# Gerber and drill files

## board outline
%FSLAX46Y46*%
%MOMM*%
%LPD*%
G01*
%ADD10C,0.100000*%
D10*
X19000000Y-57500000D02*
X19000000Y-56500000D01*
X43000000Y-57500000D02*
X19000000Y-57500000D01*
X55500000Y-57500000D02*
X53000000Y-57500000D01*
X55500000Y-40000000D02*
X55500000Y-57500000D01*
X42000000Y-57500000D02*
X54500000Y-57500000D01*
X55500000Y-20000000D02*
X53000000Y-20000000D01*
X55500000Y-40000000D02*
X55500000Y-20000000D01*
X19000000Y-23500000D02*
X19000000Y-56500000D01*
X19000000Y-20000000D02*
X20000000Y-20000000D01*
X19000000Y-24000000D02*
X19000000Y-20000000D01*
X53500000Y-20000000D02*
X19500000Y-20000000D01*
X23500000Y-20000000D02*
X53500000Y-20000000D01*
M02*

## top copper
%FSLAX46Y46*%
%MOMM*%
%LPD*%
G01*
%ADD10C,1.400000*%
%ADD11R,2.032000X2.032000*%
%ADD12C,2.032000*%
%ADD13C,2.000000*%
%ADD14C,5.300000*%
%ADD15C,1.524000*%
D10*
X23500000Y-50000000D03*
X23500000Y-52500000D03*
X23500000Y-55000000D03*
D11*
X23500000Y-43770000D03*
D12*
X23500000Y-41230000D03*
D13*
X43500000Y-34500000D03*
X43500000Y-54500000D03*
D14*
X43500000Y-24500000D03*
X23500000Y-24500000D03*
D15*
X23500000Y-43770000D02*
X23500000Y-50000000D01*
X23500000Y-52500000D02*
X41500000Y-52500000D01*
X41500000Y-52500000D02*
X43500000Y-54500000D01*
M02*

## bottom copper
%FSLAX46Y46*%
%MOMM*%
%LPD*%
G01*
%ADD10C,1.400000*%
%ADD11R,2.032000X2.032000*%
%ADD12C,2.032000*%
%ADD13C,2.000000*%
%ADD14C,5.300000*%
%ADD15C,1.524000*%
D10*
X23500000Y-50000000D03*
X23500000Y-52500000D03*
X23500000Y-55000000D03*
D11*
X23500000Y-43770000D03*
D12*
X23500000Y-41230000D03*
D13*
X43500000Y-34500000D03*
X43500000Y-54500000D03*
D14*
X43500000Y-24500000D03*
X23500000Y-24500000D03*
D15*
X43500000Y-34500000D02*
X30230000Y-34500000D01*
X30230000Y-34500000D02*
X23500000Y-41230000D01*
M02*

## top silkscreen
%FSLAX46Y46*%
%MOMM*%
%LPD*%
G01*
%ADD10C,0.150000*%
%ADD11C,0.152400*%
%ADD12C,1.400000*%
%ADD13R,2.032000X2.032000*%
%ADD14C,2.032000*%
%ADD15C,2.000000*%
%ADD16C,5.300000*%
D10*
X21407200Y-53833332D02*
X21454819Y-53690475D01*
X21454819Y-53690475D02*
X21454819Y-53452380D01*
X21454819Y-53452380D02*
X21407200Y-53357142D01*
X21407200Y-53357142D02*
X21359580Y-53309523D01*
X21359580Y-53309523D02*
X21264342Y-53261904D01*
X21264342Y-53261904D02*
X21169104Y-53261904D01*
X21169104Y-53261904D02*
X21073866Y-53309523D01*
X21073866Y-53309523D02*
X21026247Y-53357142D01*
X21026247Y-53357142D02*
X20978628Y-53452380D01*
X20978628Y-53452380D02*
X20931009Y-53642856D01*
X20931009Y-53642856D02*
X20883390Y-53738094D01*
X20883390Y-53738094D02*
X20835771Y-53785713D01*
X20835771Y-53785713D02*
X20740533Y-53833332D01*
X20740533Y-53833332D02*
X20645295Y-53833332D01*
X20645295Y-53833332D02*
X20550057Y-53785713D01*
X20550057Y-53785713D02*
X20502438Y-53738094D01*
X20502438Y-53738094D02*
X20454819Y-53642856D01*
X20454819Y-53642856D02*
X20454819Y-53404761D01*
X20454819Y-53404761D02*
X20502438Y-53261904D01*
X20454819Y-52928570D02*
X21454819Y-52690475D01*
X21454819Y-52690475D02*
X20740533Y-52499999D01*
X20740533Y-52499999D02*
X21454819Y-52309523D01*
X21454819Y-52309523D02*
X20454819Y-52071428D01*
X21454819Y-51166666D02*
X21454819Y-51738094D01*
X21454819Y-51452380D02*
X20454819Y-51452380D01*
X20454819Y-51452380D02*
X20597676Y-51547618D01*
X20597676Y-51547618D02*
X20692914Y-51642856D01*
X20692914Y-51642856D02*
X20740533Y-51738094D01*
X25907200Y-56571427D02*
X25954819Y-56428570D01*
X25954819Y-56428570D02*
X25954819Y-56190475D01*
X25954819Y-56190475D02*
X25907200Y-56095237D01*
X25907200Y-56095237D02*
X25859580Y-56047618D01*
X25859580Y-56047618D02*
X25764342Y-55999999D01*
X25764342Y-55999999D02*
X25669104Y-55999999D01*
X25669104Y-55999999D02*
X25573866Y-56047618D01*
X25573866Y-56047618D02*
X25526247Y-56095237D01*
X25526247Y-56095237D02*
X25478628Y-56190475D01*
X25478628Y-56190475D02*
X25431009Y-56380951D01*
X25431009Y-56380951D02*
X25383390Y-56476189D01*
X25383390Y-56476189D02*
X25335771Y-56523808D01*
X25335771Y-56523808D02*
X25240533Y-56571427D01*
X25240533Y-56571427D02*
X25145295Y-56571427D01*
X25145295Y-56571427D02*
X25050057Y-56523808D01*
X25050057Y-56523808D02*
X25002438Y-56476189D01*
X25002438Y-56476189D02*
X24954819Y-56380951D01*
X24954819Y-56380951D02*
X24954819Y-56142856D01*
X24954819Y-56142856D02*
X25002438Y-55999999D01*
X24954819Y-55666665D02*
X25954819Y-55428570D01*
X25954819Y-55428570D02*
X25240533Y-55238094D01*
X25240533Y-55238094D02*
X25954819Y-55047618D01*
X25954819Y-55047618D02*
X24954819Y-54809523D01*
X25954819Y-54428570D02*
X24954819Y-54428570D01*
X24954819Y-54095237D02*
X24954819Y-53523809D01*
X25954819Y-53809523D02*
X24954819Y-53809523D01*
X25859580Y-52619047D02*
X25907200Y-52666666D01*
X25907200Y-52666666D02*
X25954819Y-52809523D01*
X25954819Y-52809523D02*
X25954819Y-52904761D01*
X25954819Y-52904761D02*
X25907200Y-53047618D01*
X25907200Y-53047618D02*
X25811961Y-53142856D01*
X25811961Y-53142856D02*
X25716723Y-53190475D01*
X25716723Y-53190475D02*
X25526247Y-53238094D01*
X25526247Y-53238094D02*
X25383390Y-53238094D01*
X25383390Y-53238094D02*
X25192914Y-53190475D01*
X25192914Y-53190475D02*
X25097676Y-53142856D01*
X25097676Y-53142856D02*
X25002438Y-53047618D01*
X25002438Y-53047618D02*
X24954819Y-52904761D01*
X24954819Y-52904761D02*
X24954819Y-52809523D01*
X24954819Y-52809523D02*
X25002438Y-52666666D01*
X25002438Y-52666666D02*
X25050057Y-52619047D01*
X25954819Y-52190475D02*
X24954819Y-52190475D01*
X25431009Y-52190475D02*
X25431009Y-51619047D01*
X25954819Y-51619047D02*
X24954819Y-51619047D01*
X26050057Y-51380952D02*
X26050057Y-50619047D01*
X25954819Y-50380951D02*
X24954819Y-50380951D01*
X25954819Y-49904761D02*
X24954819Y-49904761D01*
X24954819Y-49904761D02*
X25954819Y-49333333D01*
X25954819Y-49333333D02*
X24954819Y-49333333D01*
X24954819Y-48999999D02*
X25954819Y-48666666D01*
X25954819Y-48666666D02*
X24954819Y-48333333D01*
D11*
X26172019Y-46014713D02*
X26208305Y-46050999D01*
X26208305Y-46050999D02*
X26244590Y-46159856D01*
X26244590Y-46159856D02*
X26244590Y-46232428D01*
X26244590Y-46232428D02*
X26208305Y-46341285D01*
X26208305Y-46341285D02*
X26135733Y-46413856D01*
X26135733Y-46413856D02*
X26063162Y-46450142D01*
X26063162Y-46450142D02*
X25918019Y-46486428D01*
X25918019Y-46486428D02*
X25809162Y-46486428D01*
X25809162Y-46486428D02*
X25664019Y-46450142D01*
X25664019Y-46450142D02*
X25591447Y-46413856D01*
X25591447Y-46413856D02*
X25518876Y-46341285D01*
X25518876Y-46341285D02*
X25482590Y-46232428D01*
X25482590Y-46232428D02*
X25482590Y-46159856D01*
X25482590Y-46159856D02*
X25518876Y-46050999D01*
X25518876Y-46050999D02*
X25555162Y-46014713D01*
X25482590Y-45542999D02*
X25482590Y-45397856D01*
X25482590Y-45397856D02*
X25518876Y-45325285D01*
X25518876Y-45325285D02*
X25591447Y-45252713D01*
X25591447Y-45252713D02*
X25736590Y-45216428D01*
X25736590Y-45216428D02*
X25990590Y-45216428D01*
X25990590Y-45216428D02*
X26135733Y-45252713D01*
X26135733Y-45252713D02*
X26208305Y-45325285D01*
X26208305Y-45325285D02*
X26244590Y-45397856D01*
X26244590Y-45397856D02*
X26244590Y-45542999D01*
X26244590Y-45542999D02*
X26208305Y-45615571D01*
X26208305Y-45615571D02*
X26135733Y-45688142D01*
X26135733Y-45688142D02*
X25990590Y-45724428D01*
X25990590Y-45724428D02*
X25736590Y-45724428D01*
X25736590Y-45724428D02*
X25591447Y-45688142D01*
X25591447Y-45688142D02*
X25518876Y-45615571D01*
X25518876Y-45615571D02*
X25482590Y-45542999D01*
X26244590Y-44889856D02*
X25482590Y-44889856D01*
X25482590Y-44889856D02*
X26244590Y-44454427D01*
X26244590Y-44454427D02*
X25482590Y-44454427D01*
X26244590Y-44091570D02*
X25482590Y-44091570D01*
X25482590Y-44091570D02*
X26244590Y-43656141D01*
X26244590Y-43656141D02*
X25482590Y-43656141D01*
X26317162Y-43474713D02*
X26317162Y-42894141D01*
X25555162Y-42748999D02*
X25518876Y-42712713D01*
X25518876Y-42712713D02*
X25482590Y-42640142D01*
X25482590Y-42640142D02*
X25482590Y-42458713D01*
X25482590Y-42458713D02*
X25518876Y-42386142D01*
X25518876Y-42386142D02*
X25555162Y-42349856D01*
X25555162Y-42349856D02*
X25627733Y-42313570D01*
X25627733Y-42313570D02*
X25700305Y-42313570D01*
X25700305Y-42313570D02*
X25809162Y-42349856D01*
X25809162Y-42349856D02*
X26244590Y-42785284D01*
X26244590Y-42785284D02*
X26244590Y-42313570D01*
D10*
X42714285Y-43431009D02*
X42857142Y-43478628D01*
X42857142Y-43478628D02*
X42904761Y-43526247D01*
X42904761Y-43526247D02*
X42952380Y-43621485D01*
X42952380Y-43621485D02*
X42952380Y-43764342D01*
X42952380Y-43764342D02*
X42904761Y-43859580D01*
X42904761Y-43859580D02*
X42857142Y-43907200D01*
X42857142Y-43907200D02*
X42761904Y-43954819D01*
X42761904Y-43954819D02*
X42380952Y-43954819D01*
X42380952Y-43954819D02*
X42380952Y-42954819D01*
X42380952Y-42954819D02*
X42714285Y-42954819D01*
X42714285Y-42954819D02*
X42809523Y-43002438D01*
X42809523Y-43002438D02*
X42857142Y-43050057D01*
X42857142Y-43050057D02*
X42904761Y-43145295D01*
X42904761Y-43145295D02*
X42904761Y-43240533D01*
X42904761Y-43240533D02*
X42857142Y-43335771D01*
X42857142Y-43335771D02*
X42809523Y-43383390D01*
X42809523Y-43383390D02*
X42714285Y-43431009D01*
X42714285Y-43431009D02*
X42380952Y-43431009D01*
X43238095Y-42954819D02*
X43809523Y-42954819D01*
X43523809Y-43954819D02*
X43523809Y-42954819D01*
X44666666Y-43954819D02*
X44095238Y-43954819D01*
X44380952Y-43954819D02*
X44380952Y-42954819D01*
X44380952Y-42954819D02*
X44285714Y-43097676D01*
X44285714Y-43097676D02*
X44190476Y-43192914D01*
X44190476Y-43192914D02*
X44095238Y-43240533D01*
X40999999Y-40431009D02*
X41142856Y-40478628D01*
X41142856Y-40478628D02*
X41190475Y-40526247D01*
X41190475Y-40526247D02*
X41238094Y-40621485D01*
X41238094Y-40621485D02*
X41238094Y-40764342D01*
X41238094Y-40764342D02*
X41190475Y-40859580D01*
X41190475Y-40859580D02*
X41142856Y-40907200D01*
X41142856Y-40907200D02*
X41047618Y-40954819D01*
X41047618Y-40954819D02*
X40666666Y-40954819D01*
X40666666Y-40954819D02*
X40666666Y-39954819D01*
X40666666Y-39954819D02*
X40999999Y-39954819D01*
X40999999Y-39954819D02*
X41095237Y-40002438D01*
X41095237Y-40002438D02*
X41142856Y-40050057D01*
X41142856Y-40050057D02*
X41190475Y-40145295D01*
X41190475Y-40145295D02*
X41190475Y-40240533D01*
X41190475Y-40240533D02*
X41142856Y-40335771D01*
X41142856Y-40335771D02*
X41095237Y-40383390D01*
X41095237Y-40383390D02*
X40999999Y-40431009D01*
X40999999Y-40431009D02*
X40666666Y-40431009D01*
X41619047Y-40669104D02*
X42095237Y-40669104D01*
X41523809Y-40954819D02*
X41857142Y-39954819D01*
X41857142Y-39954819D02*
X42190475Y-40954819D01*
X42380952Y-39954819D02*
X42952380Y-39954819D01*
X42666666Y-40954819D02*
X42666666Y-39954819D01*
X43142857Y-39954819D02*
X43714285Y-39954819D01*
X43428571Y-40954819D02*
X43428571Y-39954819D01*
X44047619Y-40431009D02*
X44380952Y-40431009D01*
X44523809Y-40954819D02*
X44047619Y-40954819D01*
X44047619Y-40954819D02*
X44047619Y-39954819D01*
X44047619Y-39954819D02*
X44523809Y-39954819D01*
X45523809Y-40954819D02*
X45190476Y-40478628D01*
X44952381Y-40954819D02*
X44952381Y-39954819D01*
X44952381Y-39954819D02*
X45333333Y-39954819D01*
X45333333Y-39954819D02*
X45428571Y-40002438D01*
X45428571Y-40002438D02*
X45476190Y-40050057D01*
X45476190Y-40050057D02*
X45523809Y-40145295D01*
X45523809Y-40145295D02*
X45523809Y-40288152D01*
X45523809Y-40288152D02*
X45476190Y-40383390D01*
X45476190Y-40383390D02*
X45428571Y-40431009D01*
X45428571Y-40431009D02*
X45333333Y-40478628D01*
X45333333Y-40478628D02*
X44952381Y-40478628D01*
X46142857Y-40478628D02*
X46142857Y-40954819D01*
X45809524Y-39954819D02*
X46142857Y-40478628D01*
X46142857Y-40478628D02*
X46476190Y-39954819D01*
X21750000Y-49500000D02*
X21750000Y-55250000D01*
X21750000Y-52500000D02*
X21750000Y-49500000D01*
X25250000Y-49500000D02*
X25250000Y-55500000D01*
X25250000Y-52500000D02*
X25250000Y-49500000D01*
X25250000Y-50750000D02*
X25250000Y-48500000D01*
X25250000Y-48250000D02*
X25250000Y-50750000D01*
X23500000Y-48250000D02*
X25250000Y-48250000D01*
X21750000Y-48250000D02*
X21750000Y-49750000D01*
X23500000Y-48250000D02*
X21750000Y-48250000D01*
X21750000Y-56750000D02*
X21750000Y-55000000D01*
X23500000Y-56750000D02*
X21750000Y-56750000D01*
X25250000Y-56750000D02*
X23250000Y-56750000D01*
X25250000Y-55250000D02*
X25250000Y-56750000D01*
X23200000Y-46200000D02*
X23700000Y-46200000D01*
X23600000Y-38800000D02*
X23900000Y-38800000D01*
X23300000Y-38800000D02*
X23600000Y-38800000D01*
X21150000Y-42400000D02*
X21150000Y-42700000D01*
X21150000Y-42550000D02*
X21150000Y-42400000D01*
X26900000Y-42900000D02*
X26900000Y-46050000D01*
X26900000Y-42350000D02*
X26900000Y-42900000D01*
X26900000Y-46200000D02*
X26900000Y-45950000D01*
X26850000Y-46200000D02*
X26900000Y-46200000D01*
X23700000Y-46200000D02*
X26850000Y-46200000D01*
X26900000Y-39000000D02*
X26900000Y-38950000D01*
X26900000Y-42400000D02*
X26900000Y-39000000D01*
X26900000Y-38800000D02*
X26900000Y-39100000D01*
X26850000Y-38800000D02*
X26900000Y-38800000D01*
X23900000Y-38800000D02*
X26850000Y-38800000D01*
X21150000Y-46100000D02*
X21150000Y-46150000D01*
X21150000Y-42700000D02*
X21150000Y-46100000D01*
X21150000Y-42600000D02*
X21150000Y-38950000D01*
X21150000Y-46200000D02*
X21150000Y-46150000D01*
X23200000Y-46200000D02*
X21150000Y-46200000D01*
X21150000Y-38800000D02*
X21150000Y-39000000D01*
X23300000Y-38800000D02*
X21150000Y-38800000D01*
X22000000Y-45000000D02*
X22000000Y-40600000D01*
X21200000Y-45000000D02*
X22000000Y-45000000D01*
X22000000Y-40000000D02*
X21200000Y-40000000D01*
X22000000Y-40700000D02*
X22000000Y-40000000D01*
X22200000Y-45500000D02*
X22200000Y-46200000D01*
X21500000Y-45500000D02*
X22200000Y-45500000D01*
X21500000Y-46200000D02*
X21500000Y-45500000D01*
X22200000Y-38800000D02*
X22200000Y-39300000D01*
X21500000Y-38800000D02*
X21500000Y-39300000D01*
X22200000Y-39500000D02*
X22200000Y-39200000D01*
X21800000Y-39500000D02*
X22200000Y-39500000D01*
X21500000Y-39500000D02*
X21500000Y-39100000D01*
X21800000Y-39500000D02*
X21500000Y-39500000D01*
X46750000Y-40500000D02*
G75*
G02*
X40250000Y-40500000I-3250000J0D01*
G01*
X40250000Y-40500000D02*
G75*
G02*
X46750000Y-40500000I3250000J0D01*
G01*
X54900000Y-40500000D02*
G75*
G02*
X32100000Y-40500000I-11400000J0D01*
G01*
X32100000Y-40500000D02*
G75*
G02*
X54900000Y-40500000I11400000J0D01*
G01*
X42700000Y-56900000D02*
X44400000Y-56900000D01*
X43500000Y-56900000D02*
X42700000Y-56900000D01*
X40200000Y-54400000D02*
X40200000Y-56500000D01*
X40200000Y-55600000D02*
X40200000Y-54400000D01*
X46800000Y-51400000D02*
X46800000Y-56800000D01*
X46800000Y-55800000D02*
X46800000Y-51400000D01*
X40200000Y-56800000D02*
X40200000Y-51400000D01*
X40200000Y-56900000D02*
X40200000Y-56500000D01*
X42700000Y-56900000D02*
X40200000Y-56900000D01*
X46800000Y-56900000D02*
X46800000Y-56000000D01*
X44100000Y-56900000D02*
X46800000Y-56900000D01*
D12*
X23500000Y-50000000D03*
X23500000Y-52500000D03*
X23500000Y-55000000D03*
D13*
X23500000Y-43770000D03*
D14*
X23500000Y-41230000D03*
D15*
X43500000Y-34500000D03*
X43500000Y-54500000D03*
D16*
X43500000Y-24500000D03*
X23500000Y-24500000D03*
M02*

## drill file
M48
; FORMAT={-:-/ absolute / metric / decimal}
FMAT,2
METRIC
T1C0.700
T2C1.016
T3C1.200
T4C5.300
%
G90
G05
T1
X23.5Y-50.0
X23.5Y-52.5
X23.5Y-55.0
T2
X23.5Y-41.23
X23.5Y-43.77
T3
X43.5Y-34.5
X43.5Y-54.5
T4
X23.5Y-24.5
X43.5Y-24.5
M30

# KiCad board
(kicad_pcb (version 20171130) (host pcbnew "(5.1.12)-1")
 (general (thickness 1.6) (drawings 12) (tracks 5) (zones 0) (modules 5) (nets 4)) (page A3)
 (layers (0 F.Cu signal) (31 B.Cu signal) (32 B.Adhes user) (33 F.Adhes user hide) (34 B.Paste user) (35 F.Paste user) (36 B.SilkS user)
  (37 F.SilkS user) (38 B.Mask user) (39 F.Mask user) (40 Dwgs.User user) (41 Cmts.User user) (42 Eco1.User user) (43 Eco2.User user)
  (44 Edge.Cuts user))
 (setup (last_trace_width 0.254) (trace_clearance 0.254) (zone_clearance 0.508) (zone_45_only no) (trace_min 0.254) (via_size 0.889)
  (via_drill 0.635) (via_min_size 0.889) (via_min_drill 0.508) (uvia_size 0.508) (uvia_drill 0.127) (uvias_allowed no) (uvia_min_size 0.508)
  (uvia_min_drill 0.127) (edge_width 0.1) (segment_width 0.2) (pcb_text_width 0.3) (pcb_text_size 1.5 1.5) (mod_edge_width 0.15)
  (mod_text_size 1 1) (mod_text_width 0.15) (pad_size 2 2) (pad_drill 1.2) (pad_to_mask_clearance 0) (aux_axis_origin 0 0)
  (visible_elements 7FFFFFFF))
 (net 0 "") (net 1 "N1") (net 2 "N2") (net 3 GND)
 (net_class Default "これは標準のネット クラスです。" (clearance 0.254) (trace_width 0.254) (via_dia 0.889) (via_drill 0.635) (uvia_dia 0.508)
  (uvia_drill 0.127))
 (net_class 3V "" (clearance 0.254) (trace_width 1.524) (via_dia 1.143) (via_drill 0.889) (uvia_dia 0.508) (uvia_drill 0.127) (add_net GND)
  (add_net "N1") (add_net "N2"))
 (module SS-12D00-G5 (layer F.Cu) (at 23.5 52.5 270)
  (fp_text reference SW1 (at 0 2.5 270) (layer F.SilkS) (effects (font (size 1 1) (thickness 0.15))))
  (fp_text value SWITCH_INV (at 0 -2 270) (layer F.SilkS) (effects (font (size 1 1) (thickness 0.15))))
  (fp_line (start -3 1.75) (end 2.75 1.75) (layer F.SilkS) (width 0.15))
  (fp_line (start 0 1.75) (end -3 1.75) (layer F.SilkS) (width 0.15))
  (fp_line (start -3 -1.75) (end 3 -1.75) (layer F.SilkS) (width 0.15))
  (fp_line (start 0 -1.75) (end -3 -1.75) (layer F.SilkS) (width 0.15))
  (fp_line (start -1.75 -1.75) (end -4 -1.75) (layer F.SilkS) (width 0.15))
  (fp_line (start -4.25 -1.75) (end -1.75 -1.75) (layer F.SilkS) (width 0.15))
  (fp_line (start -4.25 0) (end -4.25 -1.75) (layer F.SilkS) (width 0.15))
  (fp_line (start -4.25 1.75) (end -2.75 1.75) (layer F.SilkS) (width 0.15))
  (fp_line (start -4.25 0) (end -4.25 1.75) (layer F.SilkS) (width 0.15))
  (fp_line (start 4.25 1.75) (end 2.5 1.75) (layer F.SilkS) (width 0.15))
  (fp_line (start 4.25 0) (end 4.25 1.75) (layer F.SilkS) (width 0.15))
  (fp_line (start 4.25 -1.75) (end 4.25 0.25) (layer F.SilkS) (width 0.15))
  (fp_line (start 2.75 -1.75) (end 4.25 -1.75) (layer F.SilkS) (width 0.15))
  (pad 1 thru_hole circle (at -2.5 0 270) (size 1.4 1.4) (drill 0.7) (layers *.Cu *.Mask F.SilkS) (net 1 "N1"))
  (pad 2 thru_hole circle (at 0 0 270) (size 1.4 1.4) (drill 0.7) (layers *.Cu *.Mask F.SilkS) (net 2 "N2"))
  (pad 3 thru_hole circle (at 2.5 0 270) (size 1.4 1.4) (drill 0.7) (layers *.Cu *.Mask F.SilkS)))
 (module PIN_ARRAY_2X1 (layer F.Cu) (at 23.5 42.5 90)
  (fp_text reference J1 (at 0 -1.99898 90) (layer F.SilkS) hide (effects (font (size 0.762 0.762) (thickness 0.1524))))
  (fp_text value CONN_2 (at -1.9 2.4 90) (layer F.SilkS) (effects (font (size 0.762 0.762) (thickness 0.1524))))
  (fp_line (start -3.7 -0.3) (end -3.7 0.2) (layer F.SilkS) (width 0.15))
  (fp_line (start 3.7 0.1) (end 3.7 0.4) (layer F.SilkS) (width 0.15))
  (fp_line (start 3.7 -0.2) (end 3.7 0.1) (layer F.SilkS) (width 0.15))
  (fp_line (start 0.1 -2.35) (end -0.2 -2.35) (layer F.SilkS) (width 0.15))
  (fp_line (start -0.05 -2.35) (end 0.1 -2.35) (layer F.SilkS) (width 0.15))
  (fp_line (start -0.4 3.4) (end -3.55 3.4) (layer F.SilkS) (width 0.15))
  (fp_line (start 0.15 3.4) (end -0.4 3.4) (layer F.SilkS) (width 0.15))
  (fp_line (start -3.7 3.4) (end -3.45 3.4) (layer F.SilkS) (width 0.15))
  (fp_line (start -3.7 3.35) (end -3.7 3.4) (layer F.SilkS) (width 0.15))
  (fp_line (start -3.7 0.2) (end -3.7 3.35) (layer F.SilkS) (width 0.15))
  (fp_line (start 3.5 3.4) (end 3.55 3.4) (layer F.SilkS) (width 0.15))
  (fp_line (start 0.1 3.4) (end 3.5 3.4) (layer F.SilkS) (width 0.15))
  (fp_line (start 3.7 3.4) (end 3.4 3.4) (layer F.SilkS) (width 0.15))
  (fp_line (start 3.7 3.35) (end 3.7 3.4) (layer F.SilkS) (width 0.15))
  (fp_line (start 3.7 0.4) (end 3.7 3.35) (layer F.SilkS) (width 0.15))
  (fp_line (start -3.6 -2.35) (end -3.65 -2.35) (layer F.SilkS) (width 0.15))
  (fp_line (start -0.2 -2.35) (end -3.6 -2.35) (layer F.SilkS) (width 0.15))
  (fp_line (start -0.1 -2.35) (end 3.55 -2.35) (layer F.SilkS) (width 0.15))
  (fp_line (start -3.7 -2.35) (end -3.65 -2.35) (layer F.SilkS) (width 0.15))
  (fp_line (start -3.7 -0.3) (end -3.7 -2.35) (layer F.SilkS) (width 0.15))
  (fp_line (start 3.7 -2.35) (end 3.5 -2.35) (layer F.SilkS) (width 0.15))
  (fp_line (start 3.7 -0.2) (end 3.7 -2.35) (layer F.SilkS) (width 0.15))
  (fp_line (start -2.5 -1.5) (end 1.9 -1.5) (layer F.SilkS) (width 0.15))
  (fp_line (start -2.5 -2.3) (end -2.5 -1.5) (layer F.SilkS) (width 0.15))
  (fp_line (start 2.5 -1.5) (end 2.5 -2.3) (layer F.SilkS) (width 0.15))
  (fp_line (start 1.8 -1.5) (end 2.5 -1.5) (layer F.SilkS) (width 0.15))
  (fp_line (start -3 -1.3) (end -3.7 -1.3) (layer F.SilkS) (width 0.15))
  (fp_line (start -3 -2) (end -3 -1.3) (layer F.SilkS) (width 0.15))
  (fp_line (start -3.7 -2) (end -3 -2) (layer F.SilkS) (width 0.15))
  (fp_line (start 3.7 -1.3) (end 3.2 -1.3) (layer F.SilkS) (width 0.15))
  (fp_line (start 3.7 -2) (end 3.2 -2) (layer F.SilkS) (width 0.15))
  (fp_line (start 3 -1.3) (end 3.3 -1.3) (layer F.SilkS) (width 0.15))
  (fp_line (start 3 -1.7) (end 3 -1.3) (layer F.SilkS) (width 0.15))
  (fp_line (start 3 -2) (end 3.4 -2) (layer F.SilkS) (width 0.15))
  (fp_line (start 3 -1.7) (end 3 -2) (layer F.SilkS) (width 0.15))
  (pad 1 thru_hole rect (at -1.27 0 90) (size 2.032 2.032) (drill 1.016) (layers *.Cu *.Mask F.SilkS) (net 1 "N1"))
  (pad 2 thru_hole circle (at 1.27 0 90) (size 2.032 2.032) (drill 1.016) (layers *.Cu *.Mask F.SilkS) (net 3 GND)))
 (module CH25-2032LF (layer F.Cu) (at 43.5 40.5)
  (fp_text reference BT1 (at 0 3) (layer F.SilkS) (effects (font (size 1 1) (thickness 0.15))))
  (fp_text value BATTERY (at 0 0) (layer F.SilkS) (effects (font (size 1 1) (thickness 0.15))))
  (fp_circle (center 0 0) (end 3.25 0) (layer F.SilkS) (width 0.15))
  (fp_circle (center 0 0) (end 11.4 0) (layer F.SilkS) (width 0.15))
  (fp_line (start -0.8 16.4) (end 0.9 16.4) (layer F.SilkS) (width 0.15))
  (fp_line (start 0 16.4) (end -0.8 16.4) (layer F.SilkS) (width 0.15))
  (fp_line (start -3.3 13.9) (end -3.3 16) (layer F.SilkS) (width 0.15))
  (fp_line (start -3.3 15.1) (end -3.3 13.9) (layer F.SilkS) (width 0.15))
  (fp_line (start 3.3 10.9) (end 3.3 16.3) (layer F.SilkS) (width 0.15))
  (fp_line (start 3.3 15.3) (end 3.3 10.9) (layer F.SilkS) (width 0.15))
  (fp_line (start -3.3 16.3) (end -3.3 10.9) (layer F.SilkS) (width 0.15))
  (fp_line (start -3.3 16.4) (end -3.3 16) (layer F.SilkS) (width 0.15))
  (fp_line (start -0.8 16.4) (end -3.3 16.4) (layer F.SilkS) (width 0.15))
  (fp_line (start 3.3 16.4) (end 3.3 15.5) (layer F.SilkS) (width 0.15))
  (fp_line (start 0.6 16.4) (end 3.3 16.4) (layer F.SilkS) (width 0.15))
  (pad 2 thru_hole circle (at 0 -6) (size 2 2) (drill 1.2) (layers *.Cu *.Mask F.SilkS) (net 3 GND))
  (pad 1 thru_hole circle (at 0 14) (size 2 2) (drill 1.2) (layers *.Cu *.Mask F.SilkS) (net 2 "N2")))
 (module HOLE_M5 (layer F.Cu) (at 43.5 24.5)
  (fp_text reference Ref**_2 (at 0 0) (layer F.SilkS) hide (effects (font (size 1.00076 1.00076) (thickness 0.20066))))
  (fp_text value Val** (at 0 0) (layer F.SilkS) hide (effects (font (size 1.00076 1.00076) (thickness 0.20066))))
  (pad "" thru_hole circle (at 0 0) (size 5.3 5.3) (drill 5.3) (layers *.Cu *.Mask F.SilkS) (clearance 1.50114)))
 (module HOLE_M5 (layer F.Cu) (at 23.5 24.5)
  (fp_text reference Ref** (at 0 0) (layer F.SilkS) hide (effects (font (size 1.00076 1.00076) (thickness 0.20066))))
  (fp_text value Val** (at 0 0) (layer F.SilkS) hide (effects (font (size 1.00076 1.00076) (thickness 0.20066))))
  (pad "" thru_hole circle (at 0 0) (size 5.3 5.3) (drill 5.3) (layers *.Cu *.Mask F.SilkS) (clearance 1.50114)))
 (gr_line (start 19 57.5) (end 19 56.5) (angle 90) (layer Edge.Cuts) (width 0.1))
 (gr_line (start 43 57.5) (end 19 57.5) (angle 90) (layer Edge.Cuts) (width 0.1))
 (gr_line (start 55.5 57.5) (end 53 57.5) (angle 90) (layer Edge.Cuts) (width 0.1))
 (gr_line (start 55.5 40) (end 55.5 57.5) (angle 90) (layer Edge.Cuts) (width 0.1))
 (gr_line (start 42 57.5) (end 54.5 57.5) (angle 90) (layer Edge.Cuts) (width 0.1))
 (gr_line (start 55.5 20) (end 53 20) (angle 90) (layer Edge.Cuts) (width 0.1))
 (gr_line (start 55.5 40) (end 55.5 20) (angle 90) (layer Edge.Cuts) (width 0.1))
 (gr_line (start 19 23.5) (end 19 56.5) (angle 90) (layer Edge.Cuts) (width 0.1))
 (gr_line (start 19 20) (end 20 20) (angle 90) (layer Edge.Cuts) (width 0.1))
 (gr_line (start 19 24) (end 19 20) (angle 90) (layer Edge.Cuts) (width 0.1))
 (gr_line (start 53.5 20) (end 19.5 20) (angle 90) (layer Edge.Cuts) (width 0.1))
 (gr_line (start 23.5 20) (end 53.5 20) (angle 90) (layer Edge.Cuts) (width 0.1))
 (segment (start 43.5 34.5) (end 30.23 34.5) (width 1.524) (layer B.Cu) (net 3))
 (segment (start 30.23 34.5) (end 23.5 41.23) (width 1.524) (layer B.Cu) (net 3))
 (segment (start 23.5 43.77) (end 23.5 50) (width 1.524) (layer F.Cu) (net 1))
 (segment (start 23.5 52.5) (end 41.5 52.5) (width 1.524) (layer F.Cu) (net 2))
 (segment (start 41.5 52.5) (end 43.5 54.5) (width 1.524) (layer F.Cu) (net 2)))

